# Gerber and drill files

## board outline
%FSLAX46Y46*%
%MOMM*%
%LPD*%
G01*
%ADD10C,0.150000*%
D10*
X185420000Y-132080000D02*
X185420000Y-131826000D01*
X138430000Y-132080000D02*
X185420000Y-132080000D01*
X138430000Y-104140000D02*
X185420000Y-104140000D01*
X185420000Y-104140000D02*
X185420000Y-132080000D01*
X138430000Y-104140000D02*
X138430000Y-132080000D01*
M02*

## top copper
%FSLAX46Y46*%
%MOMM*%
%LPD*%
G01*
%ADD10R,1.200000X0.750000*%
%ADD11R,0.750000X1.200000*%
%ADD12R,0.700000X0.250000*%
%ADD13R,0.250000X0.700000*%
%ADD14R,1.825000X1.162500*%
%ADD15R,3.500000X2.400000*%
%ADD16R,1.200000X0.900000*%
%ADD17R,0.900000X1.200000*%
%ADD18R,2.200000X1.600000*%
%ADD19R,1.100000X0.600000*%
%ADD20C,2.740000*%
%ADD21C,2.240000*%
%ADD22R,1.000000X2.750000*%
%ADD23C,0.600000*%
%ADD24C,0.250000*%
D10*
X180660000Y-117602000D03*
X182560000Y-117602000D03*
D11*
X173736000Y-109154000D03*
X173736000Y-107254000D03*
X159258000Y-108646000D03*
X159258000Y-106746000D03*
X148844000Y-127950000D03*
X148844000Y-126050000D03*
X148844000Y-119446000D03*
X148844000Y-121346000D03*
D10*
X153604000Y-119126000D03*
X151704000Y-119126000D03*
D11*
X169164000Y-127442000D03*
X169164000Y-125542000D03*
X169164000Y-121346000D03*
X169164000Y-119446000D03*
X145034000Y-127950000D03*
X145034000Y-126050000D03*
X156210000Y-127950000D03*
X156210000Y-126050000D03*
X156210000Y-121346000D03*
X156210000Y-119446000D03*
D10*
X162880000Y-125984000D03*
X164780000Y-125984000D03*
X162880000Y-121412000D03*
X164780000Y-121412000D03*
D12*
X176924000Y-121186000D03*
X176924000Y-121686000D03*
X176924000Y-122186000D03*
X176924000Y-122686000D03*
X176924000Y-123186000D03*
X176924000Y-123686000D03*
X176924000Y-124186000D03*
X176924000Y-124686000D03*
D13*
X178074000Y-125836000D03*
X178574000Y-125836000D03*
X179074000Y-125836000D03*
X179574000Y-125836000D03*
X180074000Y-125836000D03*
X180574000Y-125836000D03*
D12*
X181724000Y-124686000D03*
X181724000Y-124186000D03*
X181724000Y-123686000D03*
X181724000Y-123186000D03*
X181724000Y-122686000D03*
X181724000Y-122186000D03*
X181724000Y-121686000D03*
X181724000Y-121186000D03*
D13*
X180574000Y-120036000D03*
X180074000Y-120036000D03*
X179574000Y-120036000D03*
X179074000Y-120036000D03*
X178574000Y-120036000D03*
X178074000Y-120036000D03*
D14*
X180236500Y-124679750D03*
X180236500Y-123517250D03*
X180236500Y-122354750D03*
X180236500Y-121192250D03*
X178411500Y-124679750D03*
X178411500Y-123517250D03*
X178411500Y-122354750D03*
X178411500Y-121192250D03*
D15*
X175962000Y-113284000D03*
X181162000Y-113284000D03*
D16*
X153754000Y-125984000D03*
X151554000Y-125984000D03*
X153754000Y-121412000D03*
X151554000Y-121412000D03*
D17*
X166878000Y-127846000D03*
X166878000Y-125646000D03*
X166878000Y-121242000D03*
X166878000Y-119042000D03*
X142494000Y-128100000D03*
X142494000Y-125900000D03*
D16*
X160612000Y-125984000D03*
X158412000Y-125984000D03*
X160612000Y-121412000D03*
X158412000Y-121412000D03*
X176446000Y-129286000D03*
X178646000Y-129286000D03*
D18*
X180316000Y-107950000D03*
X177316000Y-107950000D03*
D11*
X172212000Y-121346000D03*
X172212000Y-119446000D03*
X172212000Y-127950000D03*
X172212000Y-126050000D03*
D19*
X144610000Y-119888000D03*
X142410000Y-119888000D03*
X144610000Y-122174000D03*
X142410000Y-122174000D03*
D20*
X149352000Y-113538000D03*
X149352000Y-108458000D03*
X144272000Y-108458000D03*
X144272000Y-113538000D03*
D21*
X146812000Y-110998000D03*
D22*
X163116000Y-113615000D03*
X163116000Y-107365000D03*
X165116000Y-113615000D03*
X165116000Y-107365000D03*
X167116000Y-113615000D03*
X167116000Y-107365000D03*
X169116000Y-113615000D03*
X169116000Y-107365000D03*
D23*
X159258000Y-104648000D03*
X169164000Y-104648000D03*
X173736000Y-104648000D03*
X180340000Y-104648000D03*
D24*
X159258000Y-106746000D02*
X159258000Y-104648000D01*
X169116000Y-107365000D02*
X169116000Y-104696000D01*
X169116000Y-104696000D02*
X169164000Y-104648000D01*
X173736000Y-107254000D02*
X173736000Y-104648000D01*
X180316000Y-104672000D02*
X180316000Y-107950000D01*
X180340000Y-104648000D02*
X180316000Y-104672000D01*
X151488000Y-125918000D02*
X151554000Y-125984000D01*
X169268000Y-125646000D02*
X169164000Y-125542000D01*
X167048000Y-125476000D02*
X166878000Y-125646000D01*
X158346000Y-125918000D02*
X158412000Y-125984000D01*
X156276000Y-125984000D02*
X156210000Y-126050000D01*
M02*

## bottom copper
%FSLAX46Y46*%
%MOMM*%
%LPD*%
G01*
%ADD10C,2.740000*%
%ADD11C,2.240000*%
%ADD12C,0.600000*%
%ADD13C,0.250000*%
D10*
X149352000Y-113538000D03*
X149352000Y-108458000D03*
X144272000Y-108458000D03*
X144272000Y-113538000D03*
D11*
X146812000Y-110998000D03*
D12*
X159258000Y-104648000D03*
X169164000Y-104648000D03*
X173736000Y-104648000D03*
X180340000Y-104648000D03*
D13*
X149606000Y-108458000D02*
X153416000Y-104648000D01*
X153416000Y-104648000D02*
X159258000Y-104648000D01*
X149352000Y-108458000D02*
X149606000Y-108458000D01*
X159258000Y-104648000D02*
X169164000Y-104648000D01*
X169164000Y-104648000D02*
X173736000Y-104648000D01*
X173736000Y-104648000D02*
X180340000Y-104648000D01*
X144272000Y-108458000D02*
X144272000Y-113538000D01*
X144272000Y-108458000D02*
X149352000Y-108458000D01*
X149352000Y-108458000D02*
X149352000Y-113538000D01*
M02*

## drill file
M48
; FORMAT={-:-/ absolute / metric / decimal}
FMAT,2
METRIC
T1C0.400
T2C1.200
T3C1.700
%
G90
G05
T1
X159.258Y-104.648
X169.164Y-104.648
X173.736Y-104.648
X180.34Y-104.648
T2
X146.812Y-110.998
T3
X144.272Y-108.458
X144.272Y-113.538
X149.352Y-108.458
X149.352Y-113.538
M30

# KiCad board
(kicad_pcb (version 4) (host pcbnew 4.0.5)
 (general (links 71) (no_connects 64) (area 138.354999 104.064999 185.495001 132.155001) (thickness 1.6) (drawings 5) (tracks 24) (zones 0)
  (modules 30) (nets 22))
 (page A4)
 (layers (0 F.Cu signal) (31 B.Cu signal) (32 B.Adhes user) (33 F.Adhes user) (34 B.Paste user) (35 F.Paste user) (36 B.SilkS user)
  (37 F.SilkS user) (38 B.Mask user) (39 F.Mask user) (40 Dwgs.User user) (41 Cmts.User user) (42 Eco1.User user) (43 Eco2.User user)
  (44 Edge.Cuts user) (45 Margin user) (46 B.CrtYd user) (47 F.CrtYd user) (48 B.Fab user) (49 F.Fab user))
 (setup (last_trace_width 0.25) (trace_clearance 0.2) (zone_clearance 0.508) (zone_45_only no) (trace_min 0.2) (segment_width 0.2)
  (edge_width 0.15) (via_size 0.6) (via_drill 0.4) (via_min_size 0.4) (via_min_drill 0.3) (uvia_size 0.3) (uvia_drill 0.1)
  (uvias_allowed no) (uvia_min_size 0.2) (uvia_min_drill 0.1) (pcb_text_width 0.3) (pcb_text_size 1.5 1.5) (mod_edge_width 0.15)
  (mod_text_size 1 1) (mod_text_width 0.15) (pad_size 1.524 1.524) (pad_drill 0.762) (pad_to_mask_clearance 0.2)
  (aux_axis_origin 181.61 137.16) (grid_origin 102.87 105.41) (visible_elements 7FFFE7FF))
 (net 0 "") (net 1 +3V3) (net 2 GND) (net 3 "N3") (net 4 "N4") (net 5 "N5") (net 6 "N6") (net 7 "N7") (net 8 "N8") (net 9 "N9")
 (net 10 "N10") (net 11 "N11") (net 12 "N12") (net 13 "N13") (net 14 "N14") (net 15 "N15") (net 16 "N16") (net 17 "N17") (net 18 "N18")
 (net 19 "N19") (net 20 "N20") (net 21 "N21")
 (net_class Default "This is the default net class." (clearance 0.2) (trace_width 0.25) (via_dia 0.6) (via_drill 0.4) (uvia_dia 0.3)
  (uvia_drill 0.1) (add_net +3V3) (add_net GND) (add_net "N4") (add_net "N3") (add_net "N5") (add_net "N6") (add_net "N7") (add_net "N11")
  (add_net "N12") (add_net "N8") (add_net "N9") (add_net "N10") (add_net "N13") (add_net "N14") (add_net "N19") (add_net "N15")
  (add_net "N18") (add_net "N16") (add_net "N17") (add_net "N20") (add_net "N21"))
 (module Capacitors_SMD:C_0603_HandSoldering (layer F.Cu) (at 181.61 117.602)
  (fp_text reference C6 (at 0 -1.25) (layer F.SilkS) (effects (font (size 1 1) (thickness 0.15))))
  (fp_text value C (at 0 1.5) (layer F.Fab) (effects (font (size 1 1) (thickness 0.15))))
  (pad 1 smd rect (at -0.95 0) (size 1.2 0.75) (layers F.Cu F.Paste F.Mask) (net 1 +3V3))
  (pad 2 smd rect (at 0.95 0) (size 1.2 0.75) (layers F.Cu F.Paste F.Mask) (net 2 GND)))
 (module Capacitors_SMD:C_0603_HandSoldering (layer F.Cu) (at 173.736 108.204 90)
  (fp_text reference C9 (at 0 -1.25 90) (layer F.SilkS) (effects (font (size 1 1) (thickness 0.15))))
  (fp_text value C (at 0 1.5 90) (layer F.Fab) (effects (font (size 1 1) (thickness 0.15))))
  (pad 1 smd rect (at -0.95 0 90) (size 1.2 0.75) (layers F.Cu F.Paste F.Mask) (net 1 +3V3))
  (pad 2 smd rect (at 0.95 0 90) (size 1.2 0.75) (layers F.Cu F.Paste F.Mask) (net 2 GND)))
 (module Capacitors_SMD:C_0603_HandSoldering (layer F.Cu) (at 159.258 107.696 90)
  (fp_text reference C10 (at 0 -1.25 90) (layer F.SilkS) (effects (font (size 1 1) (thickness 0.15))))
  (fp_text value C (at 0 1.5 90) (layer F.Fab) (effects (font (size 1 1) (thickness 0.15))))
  (pad 1 smd rect (at -0.95 0 90) (size 1.2 0.75) (layers F.Cu F.Paste F.Mask) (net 1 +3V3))
  (pad 2 smd rect (at 0.95 0 90) (size 1.2 0.75) (layers F.Cu F.Paste F.Mask) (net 2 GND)))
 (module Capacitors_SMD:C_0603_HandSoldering (layer F.Cu) (at 148.844 127 90)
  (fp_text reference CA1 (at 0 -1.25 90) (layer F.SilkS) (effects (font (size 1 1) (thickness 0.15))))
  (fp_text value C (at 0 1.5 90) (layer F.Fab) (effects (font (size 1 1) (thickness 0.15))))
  (pad 1 smd rect (at -0.95 0 90) (size 1.2 0.75) (layers F.Cu F.Paste F.Mask) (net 2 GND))
  (pad 2 smd rect (at 0.95 0 90) (size 1.2 0.75) (layers F.Cu F.Paste F.Mask) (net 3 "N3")))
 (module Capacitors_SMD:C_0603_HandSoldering (layer F.Cu) (at 148.844 120.396 270)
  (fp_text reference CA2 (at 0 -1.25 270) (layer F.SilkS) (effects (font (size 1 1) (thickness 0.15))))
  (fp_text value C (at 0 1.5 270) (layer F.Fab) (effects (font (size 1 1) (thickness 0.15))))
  (pad 1 smd rect (at -0.95 0 270) (size 1.2 0.75) (layers F.Cu F.Paste F.Mask) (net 2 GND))
  (pad 2 smd rect (at 0.95 0 270) (size 1.2 0.75) (layers F.Cu F.Paste F.Mask) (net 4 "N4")))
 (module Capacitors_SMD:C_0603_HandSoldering (layer F.Cu) (at 152.654 119.126 180)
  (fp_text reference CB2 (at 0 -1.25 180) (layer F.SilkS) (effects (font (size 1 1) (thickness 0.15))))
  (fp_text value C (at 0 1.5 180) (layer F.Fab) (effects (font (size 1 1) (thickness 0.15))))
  (pad 1 smd rect (at -0.95 0 180) (size 1.2 0.75) (layers F.Cu F.Paste F.Mask) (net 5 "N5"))
  (pad 2 smd rect (at 0.95 0 180) (size 1.2 0.75) (layers F.Cu F.Paste F.Mask) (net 3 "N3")))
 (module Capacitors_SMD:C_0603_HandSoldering (layer F.Cu) (at 169.164 126.492 90)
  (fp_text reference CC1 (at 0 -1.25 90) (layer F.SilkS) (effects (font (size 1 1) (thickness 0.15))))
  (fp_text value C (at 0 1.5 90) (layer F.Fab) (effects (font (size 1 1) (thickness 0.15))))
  (pad 1 smd rect (at -0.95 0 90) (size 1.2 0.75) (layers F.Cu F.Paste F.Mask) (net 2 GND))
  (pad 2 smd rect (at 0.95 0 90) (size 1.2 0.75) (layers F.Cu F.Paste F.Mask) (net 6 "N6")))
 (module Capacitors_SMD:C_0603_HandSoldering (layer F.Cu) (at 169.164 120.396 90)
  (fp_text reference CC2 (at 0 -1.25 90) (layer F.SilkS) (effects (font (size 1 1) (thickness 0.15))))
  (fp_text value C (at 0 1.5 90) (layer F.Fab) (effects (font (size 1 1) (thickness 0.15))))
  (pad 1 smd rect (at -0.95 0 90) (size 1.2 0.75) (layers F.Cu F.Paste F.Mask) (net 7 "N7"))
  (pad 2 smd rect (at 0.95 0 90) (size 1.2 0.75) (layers F.Cu F.Paste F.Mask) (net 2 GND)))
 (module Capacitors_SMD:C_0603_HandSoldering (layer F.Cu) (at 145.034 127 90)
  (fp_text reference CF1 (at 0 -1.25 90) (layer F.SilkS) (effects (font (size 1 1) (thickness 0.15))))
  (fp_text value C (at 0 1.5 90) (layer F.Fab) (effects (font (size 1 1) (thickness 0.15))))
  (pad 1 smd rect (at -0.95 0 90) (size 1.2 0.75) (layers F.Cu F.Paste F.Mask) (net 4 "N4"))
  (pad 2 smd rect (at 0.95 0 90) (size 1.2 0.75) (layers F.Cu F.Paste F.Mask) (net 3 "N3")))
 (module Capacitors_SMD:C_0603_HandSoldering (layer F.Cu) (at 156.21 127 90)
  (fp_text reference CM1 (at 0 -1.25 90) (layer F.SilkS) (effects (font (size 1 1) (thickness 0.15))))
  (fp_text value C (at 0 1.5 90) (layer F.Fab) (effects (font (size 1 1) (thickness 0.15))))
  (pad 1 smd rect (at -0.95 0 90) (size 1.2 0.75) (layers F.Cu F.Paste F.Mask) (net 2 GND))
  (pad 2 smd rect (at 0.95 0 90) (size 1.2 0.75) (layers F.Cu F.Paste F.Mask) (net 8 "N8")))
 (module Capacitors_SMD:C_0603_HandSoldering (layer F.Cu) (at 156.21 120.396 90)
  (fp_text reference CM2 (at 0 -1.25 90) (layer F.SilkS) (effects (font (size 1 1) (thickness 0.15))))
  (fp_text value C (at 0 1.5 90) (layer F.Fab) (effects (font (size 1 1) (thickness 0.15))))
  (pad 1 smd rect (at -0.95 0 90) (size 1.2 0.75) (layers F.Cu F.Paste F.Mask) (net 5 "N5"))
  (pad 2 smd rect (at 0.95 0 90) (size 1.2 0.75) (layers F.Cu F.Paste F.Mask) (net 2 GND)))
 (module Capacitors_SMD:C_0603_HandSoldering (layer F.Cu) (at 163.83 125.984)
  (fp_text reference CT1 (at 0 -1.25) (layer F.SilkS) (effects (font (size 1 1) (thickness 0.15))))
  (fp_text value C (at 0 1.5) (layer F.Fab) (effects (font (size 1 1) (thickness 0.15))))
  (pad 1 smd rect (at -0.95 0) (size 1.2 0.75) (layers F.Cu F.Paste F.Mask) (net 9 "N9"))
  (pad 2 smd rect (at 0.95 0) (size 1.2 0.75) (layers F.Cu F.Paste F.Mask) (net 6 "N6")))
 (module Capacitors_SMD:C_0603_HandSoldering (layer F.Cu) (at 163.83 121.412)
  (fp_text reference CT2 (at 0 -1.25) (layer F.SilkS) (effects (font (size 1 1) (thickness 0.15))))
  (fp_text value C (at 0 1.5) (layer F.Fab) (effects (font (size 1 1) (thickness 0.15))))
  (pad 1 smd rect (at -0.95 0) (size 1.2 0.75) (layers F.Cu F.Paste F.Mask) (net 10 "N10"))
  (pad 2 smd rect (at 0.95 0) (size 1.2 0.75) (layers F.Cu F.Paste F.Mask) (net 7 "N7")))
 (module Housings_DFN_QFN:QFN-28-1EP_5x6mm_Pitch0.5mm (layer F.Cu) (at 179.324 122.936)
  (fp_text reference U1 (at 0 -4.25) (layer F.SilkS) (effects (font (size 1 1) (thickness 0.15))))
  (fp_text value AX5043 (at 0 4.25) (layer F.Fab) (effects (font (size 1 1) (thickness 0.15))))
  (pad 1 smd rect (at -2.4 -1.75) (size 0.7 0.25) (layers F.Cu F.Paste F.Mask) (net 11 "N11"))
  (pad 2 smd rect (at -2.4 -1.25) (size 0.7 0.25) (layers F.Cu F.Paste F.Mask) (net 2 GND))
  (pad 3 smd rect (at -2.4 -0.75) (size 0.7 0.25) (layers F.Cu F.Paste F.Mask) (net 6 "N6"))
  (pad 4 smd rect (at -2.4 -0.25) (size 0.7 0.25) (layers F.Cu F.Paste F.Mask) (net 7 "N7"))
  (pad 5 smd rect (at -2.4 0.25) (size 0.7 0.25) (layers F.Cu F.Paste F.Mask))
  (pad 6 smd rect (at -2.4 0.75) (size 0.7 0.25) (layers F.Cu F.Paste F.Mask) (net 2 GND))
  (pad 7 smd rect (at -2.4 1.25) (size 0.7 0.25) (layers F.Cu F.Paste F.Mask) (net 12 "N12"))
  (pad 8 smd rect (at -2.4 1.75) (size 0.7 0.25) (layers F.Cu F.Paste F.Mask))
  (pad 9 smd rect (at -1.25 2.9 90) (size 0.7 0.25) (layers F.Cu F.Paste F.Mask) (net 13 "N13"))
  (pad 10 smd rect (at -0.75 2.9 90) (size 0.7 0.25) (layers F.Cu F.Paste F.Mask) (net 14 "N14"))
  (pad 11 smd rect (at -0.25 2.9 90) (size 0.7 0.25) (layers F.Cu F.Paste F.Mask))
  (pad 12 smd rect (at 0.25 2.9 90) (size 0.7 0.25) (layers F.Cu F.Paste F.Mask))
  (pad 13 smd rect (at 0.75 2.9 90) (size 0.7 0.25) (layers F.Cu F.Paste F.Mask))
  (pad 14 smd rect (at 1.25 2.9 90) (size 0.7 0.25) (layers F.Cu F.Paste F.Mask) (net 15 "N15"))
  (pad 15 smd rect (at 2.4 1.75) (size 0.7 0.25) (layers F.Cu F.Paste F.Mask) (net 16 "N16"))
  (pad 16 smd rect (at 2.4 1.25) (size 0.7 0.25) (layers F.Cu F.Paste F.Mask) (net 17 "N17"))
  (pad 17 smd rect (at 2.4 0.75) (size 0.7 0.25) (layers F.Cu F.Paste F.Mask) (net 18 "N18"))
  (pad 18 smd rect (at 2.4 0.25) (size 0.7 0.25) (layers F.Cu F.Paste F.Mask))
  (pad 19 smd rect (at 2.4 -0.25) (size 0.7 0.25) (layers F.Cu F.Paste F.Mask) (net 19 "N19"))
  (pad 20 smd rect (at 2.4 -0.75) (size 0.7 0.25) (layers F.Cu F.Paste F.Mask))
  (pad 21 smd rect (at 2.4 -1.25) (size 0.7 0.25) (layers F.Cu F.Paste F.Mask))
  (pad 22 smd rect (at 2.4 -1.75) (size 0.7 0.25) (layers F.Cu F.Paste F.Mask))
  (pad 23 smd rect (at 1.25 -2.9 90) (size 0.7 0.25) (layers F.Cu F.Paste F.Mask) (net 1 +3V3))
  (pad 24 smd rect (at 0.75 -2.9 90) (size 0.7 0.25) (layers F.Cu F.Paste F.Mask))
  (pad 25 smd rect (at 0.25 -2.9 90) (size 0.7 0.25) (layers F.Cu F.Paste F.Mask) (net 2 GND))
  (pad 26 smd rect (at -0.25 -2.9 90) (size 0.7 0.25) (layers F.Cu F.Paste F.Mask) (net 2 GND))
  (pad 27 smd rect (at -0.75 -2.9 90) (size 0.7 0.25) (layers F.Cu F.Paste F.Mask) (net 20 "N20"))
  (pad 28 smd rect (at -1.25 -2.9 90) (size 0.7 0.25) (layers F.Cu F.Paste F.Mask) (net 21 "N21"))
  (pad 29 smd rect (at 0.9125 1.74375) (size 1.825 1.1625) (layers F.Cu F.Paste F.Mask) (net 2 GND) (solder_paste_margin_ratio -0.2))
  (pad 29 smd rect (at 0.9125 0.58125) (size 1.825 1.1625) (layers F.Cu F.Paste F.Mask) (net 2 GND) (solder_paste_margin_ratio -0.2))
  (pad 29 smd rect (at 0.9125 -0.58125) (size 1.825 1.1625) (layers F.Cu F.Paste F.Mask) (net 2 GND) (solder_paste_margin_ratio -0.2))
  (pad 29 smd rect (at 0.9125 -1.74375) (size 1.825 1.1625) (layers F.Cu F.Paste F.Mask) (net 2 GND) (solder_paste_margin_ratio -0.2))
  (pad 29 smd rect (at -0.9125 1.74375) (size 1.825 1.1625) (layers F.Cu F.Paste F.Mask) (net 2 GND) (solder_paste_margin_ratio -0.2))
  (pad 29 smd rect (at -0.9125 0.58125) (size 1.825 1.1625) (layers F.Cu F.Paste F.Mask) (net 2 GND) (solder_paste_margin_ratio -0.2))
  (pad 29 smd rect (at -0.9125 -0.58125) (size 1.825 1.1625) (layers F.Cu F.Paste F.Mask) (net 2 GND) (solder_paste_margin_ratio -0.2))
  (pad 29 smd rect (at -0.9125 -1.74375) (size 1.825 1.1625) (layers F.Cu F.Paste F.Mask) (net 2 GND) (solder_paste_margin_ratio -0.2)))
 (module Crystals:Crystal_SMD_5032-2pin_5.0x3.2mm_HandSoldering (layer F.Cu) (at 178.562 113.284)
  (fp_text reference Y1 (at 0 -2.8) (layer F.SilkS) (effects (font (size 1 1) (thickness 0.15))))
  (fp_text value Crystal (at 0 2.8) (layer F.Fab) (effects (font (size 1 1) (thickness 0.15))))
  (pad 1 smd rect (at -2.6 0) (size 3.5 2.4) (layers F.Cu F.Mask) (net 21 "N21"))
  (pad 2 smd rect (at 2.6 0) (size 3.5 2.4) (layers F.Cu F.Mask) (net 20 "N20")))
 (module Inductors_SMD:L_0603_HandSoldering (layer F.Cu) (at 152.654 125.984 180)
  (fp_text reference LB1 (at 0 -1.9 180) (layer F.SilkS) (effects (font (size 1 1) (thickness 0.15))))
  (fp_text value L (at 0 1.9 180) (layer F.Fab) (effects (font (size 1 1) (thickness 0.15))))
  (pad 1 smd rect (at -1.1 0 180) (size 1.2 0.9) (layers F.Cu F.Paste F.Mask) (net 8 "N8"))
  (pad 2 smd rect (at 1.1 0 180) (size 1.2 0.9) (layers F.Cu F.Paste F.Mask) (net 3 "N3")))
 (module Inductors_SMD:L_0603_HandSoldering (layer F.Cu) (at 152.654 121.412 180)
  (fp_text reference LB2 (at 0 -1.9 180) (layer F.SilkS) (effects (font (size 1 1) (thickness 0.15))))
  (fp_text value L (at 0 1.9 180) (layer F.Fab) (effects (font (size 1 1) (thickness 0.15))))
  (pad 1 smd rect (at -1.1 0 180) (size 1.2 0.9) (layers F.Cu F.Paste F.Mask) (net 5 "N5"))
  (pad 2 smd rect (at 1.1 0 180) (size 1.2 0.9) (layers F.Cu F.Paste F.Mask) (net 2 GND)))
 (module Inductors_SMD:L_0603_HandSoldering (layer F.Cu) (at 166.878 126.746 90)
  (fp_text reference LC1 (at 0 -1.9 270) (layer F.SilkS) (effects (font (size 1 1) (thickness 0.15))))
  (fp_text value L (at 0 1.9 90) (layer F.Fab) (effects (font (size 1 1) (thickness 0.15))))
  (pad 1 smd rect (at -1.1 0 90) (size 1.2 0.9) (layers F.Cu F.Paste F.Mask) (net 2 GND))
  (pad 2 smd rect (at 1.1 0 90) (size 1.2 0.9) (layers F.Cu F.Paste F.Mask) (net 6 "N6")))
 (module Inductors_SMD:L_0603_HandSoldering (layer F.Cu) (at 166.878 120.142 90)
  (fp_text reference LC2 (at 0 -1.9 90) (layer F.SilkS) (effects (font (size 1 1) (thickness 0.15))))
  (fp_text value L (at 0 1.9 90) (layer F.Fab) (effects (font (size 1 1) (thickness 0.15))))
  (pad 1 smd rect (at -1.1 0 90) (size 1.2 0.9) (layers F.Cu F.Paste F.Mask) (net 7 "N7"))
  (pad 2 smd rect (at 1.1 0 90) (size 1.2 0.9) (layers F.Cu F.Paste F.Mask) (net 2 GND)))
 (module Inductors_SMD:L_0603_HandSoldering (layer F.Cu) (at 142.494 127 90)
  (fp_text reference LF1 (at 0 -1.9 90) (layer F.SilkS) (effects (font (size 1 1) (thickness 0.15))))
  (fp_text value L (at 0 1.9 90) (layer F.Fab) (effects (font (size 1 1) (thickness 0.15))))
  (pad 1 smd rect (at -1.1 0 90) (size 1.2 0.9) (layers F.Cu F.Paste F.Mask) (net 4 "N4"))
  (pad 2 smd rect (at 1.1 0 90) (size 1.2 0.9) (layers F.Cu F.Paste F.Mask) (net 3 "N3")))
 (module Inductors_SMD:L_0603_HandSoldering (layer F.Cu) (at 159.512 125.984 180)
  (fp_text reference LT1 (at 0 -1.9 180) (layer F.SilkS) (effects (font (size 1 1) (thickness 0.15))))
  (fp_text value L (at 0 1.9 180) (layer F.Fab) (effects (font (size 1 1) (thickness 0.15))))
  (pad 1 smd rect (at -1.1 0 180) (size 1.2 0.9) (layers F.Cu F.Paste F.Mask) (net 9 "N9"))
  (pad 2 smd rect (at 1.1 0 180) (size 1.2 0.9) (layers F.Cu F.Paste F.Mask) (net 8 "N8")))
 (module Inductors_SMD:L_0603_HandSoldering (layer F.Cu) (at 159.512 121.412 180)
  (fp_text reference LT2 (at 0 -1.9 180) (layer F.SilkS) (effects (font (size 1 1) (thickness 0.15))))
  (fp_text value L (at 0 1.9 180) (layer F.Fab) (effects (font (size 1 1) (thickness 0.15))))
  (pad 1 smd rect (at -1.1 0 180) (size 1.2 0.9) (layers F.Cu F.Paste F.Mask) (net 10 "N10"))
  (pad 2 smd rect (at 1.1 0 180) (size 1.2 0.9) (layers F.Cu F.Paste F.Mask) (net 5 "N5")))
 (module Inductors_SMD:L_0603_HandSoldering (layer F.Cu) (at 177.546 129.286)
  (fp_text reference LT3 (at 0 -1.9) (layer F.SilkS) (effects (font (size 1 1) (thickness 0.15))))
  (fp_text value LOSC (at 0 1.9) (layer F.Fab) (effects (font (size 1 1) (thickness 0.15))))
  (pad 1 smd rect (at -1.1 0) (size 1.2 0.9) (layers F.Cu F.Paste F.Mask) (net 13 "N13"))
  (pad 2 smd rect (at 1.1 0) (size 1.2 0.9) (layers F.Cu F.Paste F.Mask) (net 14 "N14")))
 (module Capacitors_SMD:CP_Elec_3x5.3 (layer F.Cu) (at 178.816 107.95)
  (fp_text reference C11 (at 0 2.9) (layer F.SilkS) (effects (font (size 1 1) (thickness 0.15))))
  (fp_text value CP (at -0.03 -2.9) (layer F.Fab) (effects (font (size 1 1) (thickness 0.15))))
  (pad 2 smd rect (at 1.5 0) (size 2.2 1.6) (layers F.Cu F.Paste F.Mask) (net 2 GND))
  (pad 1 smd rect (at -1.5 0) (size 2.2 1.6) (layers F.Cu F.Paste F.Mask) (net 1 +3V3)))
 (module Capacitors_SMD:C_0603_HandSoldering (layer F.Cu) (at 172.212 120.396 90)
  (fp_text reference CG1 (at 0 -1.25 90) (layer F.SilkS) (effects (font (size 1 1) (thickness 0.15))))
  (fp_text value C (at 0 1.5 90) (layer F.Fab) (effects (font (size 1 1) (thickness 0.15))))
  (pad 1 smd rect (at -0.95 0 90) (size 1.2 0.75) (layers F.Cu F.Paste F.Mask) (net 11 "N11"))
  (pad 2 smd rect (at 0.95 0 90) (size 1.2 0.75) (layers F.Cu F.Paste F.Mask) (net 2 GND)))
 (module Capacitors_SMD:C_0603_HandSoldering (layer F.Cu) (at 172.212 127 90)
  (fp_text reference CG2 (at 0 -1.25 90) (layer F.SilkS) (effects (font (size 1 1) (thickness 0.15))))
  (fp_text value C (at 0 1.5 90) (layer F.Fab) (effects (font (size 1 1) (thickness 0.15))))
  (pad 1 smd rect (at -0.95 0 90) (size 1.2 0.75) (layers F.Cu F.Paste F.Mask) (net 2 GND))
  (pad 2 smd rect (at 0.95 0 90) (size 1.2 0.75) (layers F.Cu F.Paste F.Mask) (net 12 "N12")))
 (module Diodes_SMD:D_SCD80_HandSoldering (layer F.Cu) (at 143.51 119.888)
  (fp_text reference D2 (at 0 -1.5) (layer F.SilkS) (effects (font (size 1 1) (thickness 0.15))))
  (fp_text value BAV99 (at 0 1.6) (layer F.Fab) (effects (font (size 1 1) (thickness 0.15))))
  (pad 2 smd rect (at 1.1 0) (size 1.1 0.6) (layers F.Cu F.Paste F.Mask) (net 3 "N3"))
  (pad 1 smd rect (at -1.1 0) (size 1.1 0.6) (layers F.Cu F.Paste F.Mask) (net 1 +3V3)))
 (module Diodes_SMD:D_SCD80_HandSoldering (layer F.Cu) (at 143.51 122.174)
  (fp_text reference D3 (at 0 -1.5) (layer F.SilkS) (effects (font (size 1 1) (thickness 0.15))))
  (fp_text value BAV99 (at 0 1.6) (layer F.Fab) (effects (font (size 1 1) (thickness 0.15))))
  (pad 2 smd rect (at 1.1 0) (size 1.1 0.6) (layers F.Cu F.Paste F.Mask) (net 1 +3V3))
  (pad 1 smd rect (at -1.1 0) (size 1.1 0.6) (layers F.Cu F.Paste F.Mask) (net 3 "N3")))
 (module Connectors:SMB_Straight (layer F.Cu) (at 146.812 110.998 90)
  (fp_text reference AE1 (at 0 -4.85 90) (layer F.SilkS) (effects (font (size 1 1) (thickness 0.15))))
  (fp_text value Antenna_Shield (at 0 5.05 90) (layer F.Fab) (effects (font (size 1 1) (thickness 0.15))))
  (pad 2 thru_hole circle (at -2.54 2.54 90) (size 2.74 2.74) (drill 1.7) (layers *.Cu *.Mask) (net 2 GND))
  (pad 2 thru_hole circle (at 2.54 2.54 90) (size 2.74 2.74) (drill 1.7) (layers *.Cu *.Mask) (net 2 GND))
  (pad 2 thru_hole circle (at 2.54 -2.54 90) (size 2.74 2.74) (drill 1.7) (layers *.Cu *.Mask) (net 2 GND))
  (pad 2 thru_hole circle (at -2.54 -2.54 90) (size 2.74 2.74) (drill 1.7) (layers *.Cu *.Mask) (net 2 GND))
  (pad 1 thru_hole circle (at 0 0 90) (size 2.24 2.24) (drill 1.2) (layers *.Cu *.Mask) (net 4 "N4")))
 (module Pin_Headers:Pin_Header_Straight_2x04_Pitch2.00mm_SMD (layer F.Cu) (at 166.116 110.49 90)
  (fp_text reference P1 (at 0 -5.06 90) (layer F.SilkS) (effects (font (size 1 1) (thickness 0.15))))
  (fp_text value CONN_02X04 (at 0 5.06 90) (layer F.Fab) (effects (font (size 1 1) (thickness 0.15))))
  (pad 1 smd rect (at -3.125 -3 90) (size 2.75 1) (layers F.Cu F.Mask) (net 1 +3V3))
  (pad 2 smd rect (at 3.125 -3 90) (size 2.75 1) (layers F.Cu F.Mask))
  (pad 3 smd rect (at -3.125 -1 90) (size 2.75 1) (layers F.Cu F.Mask) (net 19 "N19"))
  (pad 4 smd rect (at 3.125 -1 90) (size 2.75 1) (layers F.Cu F.Mask) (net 15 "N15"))
  (pad 5 smd rect (at -3.125 1 90) (size 2.75 1) (layers F.Cu F.Mask) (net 18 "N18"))
  (pad 6 smd rect (at 3.125 1 90) (size 2.75 1) (layers F.Cu F.Mask) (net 16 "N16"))
  (pad 7 smd rect (at -3.125 3 90) (size 2.75 1) (layers F.Cu F.Mask) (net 17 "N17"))
  (pad 8 smd rect (at 3.125 3 90) (size 2.75 1) (layers F.Cu F.Mask) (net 2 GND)))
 (gr_line (start 185.42 132.08) (end 185.42 131.826) (angle 90) (layer Edge.Cuts) (width 0.15))
 (gr_line (start 138.43 132.08) (end 185.42 132.08) (angle 90) (layer Edge.Cuts) (width 0.15))
 (gr_line (start 138.43 104.14) (end 185.42 104.14) (angle 90) (layer Edge.Cuts) (width 0.15))
 (gr_line (start 185.42 104.14) (end 185.42 132.08) (angle 90) (layer Edge.Cuts) (width 0.15))
 (gr_line (start 138.43 104.14) (end 138.43 132.08) (angle 90) (layer Edge.Cuts) (width 0.15))
 (segment (start 149.606 108.458) (end 153.416 104.648) (width 0.25) (layer B.Cu) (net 2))
 (segment (start 153.416 104.648) (end 159.258 104.648) (width 0.25) (layer B.Cu) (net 2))
 (segment (start 159.258 106.746) (end 159.258 104.648) (width 0.25) (layer F.Cu) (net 2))
 (via (at 159.258 104.648) (size 0.6) (drill 0.4) (layers F.Cu B.Cu) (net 2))
 (segment (start 169.116 107.365) (end 169.116 104.696) (width 0.25) (layer F.Cu) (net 2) (status 10))
 (via (at 169.164 104.648) (size 0.6) (drill 0.4) (layers F.Cu B.Cu) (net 2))
 (segment (start 169.116 104.696) (end 169.164 104.648) (width 0.25) (layer F.Cu) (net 2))
 (segment (start 173.736 107.254) (end 173.736 104.648) (width 0.25) (layer F.Cu) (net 2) (status 10))
 (via (at 173.736 104.648) (size 0.6) (drill 0.4) (layers F.Cu B.Cu) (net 2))
 (segment (start 149.352 108.458) (end 149.606 108.458) (width 0.25) (layer B.Cu) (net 2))
 (segment (start 180.316 104.672) (end 180.316 107.95) (width 0.25) (layer F.Cu) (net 2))
 (segment (start 180.34 104.648) (end 180.316 104.672) (width 0.25) (layer F.Cu) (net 2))
 (via (at 180.34 104.648) (size 0.6) (drill 0.4) (layers F.Cu B.Cu) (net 2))
 (segment (start 159.258 104.648) (end 169.164 104.648) (width 0.25) (layer B.Cu) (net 2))
 (segment (start 169.164 104.648) (end 173.736 104.648) (width 0.25) (layer B.Cu) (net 2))
 (segment (start 173.736 104.648) (end 180.34 104.648) (width 0.25) (layer B.Cu) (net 2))
 (segment (start 144.272 108.458) (end 144.272 113.538) (width 0.25) (layer B.Cu) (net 2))
 (segment (start 144.272 108.458) (end 149.352 108.458) (width 0.25) (layer B.Cu) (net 2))
 (segment (start 149.352 108.458) (end 149.352 113.538) (width 0.25) (layer B.Cu) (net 2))
 (segment (start 151.488 125.918) (end 151.554 125.984) (width 0.25) (layer F.Cu) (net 3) (status 30))
 (segment (start 169.268 125.646) (end 169.164 125.542) (width 0.25) (layer F.Cu) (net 6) (status 30))
 (segment (start 167.048 125.476) (end 166.878 125.646) (width 0.25) (layer F.Cu) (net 6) (status 30))
 (segment (start 158.346 125.918) (end 158.412 125.984) (width 0.25) (layer F.Cu) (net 8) (status 30))
 (segment (start 156.276 125.984) (end 156.21 126.05) (width 0.25) (layer F.Cu) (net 8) (status 30)))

